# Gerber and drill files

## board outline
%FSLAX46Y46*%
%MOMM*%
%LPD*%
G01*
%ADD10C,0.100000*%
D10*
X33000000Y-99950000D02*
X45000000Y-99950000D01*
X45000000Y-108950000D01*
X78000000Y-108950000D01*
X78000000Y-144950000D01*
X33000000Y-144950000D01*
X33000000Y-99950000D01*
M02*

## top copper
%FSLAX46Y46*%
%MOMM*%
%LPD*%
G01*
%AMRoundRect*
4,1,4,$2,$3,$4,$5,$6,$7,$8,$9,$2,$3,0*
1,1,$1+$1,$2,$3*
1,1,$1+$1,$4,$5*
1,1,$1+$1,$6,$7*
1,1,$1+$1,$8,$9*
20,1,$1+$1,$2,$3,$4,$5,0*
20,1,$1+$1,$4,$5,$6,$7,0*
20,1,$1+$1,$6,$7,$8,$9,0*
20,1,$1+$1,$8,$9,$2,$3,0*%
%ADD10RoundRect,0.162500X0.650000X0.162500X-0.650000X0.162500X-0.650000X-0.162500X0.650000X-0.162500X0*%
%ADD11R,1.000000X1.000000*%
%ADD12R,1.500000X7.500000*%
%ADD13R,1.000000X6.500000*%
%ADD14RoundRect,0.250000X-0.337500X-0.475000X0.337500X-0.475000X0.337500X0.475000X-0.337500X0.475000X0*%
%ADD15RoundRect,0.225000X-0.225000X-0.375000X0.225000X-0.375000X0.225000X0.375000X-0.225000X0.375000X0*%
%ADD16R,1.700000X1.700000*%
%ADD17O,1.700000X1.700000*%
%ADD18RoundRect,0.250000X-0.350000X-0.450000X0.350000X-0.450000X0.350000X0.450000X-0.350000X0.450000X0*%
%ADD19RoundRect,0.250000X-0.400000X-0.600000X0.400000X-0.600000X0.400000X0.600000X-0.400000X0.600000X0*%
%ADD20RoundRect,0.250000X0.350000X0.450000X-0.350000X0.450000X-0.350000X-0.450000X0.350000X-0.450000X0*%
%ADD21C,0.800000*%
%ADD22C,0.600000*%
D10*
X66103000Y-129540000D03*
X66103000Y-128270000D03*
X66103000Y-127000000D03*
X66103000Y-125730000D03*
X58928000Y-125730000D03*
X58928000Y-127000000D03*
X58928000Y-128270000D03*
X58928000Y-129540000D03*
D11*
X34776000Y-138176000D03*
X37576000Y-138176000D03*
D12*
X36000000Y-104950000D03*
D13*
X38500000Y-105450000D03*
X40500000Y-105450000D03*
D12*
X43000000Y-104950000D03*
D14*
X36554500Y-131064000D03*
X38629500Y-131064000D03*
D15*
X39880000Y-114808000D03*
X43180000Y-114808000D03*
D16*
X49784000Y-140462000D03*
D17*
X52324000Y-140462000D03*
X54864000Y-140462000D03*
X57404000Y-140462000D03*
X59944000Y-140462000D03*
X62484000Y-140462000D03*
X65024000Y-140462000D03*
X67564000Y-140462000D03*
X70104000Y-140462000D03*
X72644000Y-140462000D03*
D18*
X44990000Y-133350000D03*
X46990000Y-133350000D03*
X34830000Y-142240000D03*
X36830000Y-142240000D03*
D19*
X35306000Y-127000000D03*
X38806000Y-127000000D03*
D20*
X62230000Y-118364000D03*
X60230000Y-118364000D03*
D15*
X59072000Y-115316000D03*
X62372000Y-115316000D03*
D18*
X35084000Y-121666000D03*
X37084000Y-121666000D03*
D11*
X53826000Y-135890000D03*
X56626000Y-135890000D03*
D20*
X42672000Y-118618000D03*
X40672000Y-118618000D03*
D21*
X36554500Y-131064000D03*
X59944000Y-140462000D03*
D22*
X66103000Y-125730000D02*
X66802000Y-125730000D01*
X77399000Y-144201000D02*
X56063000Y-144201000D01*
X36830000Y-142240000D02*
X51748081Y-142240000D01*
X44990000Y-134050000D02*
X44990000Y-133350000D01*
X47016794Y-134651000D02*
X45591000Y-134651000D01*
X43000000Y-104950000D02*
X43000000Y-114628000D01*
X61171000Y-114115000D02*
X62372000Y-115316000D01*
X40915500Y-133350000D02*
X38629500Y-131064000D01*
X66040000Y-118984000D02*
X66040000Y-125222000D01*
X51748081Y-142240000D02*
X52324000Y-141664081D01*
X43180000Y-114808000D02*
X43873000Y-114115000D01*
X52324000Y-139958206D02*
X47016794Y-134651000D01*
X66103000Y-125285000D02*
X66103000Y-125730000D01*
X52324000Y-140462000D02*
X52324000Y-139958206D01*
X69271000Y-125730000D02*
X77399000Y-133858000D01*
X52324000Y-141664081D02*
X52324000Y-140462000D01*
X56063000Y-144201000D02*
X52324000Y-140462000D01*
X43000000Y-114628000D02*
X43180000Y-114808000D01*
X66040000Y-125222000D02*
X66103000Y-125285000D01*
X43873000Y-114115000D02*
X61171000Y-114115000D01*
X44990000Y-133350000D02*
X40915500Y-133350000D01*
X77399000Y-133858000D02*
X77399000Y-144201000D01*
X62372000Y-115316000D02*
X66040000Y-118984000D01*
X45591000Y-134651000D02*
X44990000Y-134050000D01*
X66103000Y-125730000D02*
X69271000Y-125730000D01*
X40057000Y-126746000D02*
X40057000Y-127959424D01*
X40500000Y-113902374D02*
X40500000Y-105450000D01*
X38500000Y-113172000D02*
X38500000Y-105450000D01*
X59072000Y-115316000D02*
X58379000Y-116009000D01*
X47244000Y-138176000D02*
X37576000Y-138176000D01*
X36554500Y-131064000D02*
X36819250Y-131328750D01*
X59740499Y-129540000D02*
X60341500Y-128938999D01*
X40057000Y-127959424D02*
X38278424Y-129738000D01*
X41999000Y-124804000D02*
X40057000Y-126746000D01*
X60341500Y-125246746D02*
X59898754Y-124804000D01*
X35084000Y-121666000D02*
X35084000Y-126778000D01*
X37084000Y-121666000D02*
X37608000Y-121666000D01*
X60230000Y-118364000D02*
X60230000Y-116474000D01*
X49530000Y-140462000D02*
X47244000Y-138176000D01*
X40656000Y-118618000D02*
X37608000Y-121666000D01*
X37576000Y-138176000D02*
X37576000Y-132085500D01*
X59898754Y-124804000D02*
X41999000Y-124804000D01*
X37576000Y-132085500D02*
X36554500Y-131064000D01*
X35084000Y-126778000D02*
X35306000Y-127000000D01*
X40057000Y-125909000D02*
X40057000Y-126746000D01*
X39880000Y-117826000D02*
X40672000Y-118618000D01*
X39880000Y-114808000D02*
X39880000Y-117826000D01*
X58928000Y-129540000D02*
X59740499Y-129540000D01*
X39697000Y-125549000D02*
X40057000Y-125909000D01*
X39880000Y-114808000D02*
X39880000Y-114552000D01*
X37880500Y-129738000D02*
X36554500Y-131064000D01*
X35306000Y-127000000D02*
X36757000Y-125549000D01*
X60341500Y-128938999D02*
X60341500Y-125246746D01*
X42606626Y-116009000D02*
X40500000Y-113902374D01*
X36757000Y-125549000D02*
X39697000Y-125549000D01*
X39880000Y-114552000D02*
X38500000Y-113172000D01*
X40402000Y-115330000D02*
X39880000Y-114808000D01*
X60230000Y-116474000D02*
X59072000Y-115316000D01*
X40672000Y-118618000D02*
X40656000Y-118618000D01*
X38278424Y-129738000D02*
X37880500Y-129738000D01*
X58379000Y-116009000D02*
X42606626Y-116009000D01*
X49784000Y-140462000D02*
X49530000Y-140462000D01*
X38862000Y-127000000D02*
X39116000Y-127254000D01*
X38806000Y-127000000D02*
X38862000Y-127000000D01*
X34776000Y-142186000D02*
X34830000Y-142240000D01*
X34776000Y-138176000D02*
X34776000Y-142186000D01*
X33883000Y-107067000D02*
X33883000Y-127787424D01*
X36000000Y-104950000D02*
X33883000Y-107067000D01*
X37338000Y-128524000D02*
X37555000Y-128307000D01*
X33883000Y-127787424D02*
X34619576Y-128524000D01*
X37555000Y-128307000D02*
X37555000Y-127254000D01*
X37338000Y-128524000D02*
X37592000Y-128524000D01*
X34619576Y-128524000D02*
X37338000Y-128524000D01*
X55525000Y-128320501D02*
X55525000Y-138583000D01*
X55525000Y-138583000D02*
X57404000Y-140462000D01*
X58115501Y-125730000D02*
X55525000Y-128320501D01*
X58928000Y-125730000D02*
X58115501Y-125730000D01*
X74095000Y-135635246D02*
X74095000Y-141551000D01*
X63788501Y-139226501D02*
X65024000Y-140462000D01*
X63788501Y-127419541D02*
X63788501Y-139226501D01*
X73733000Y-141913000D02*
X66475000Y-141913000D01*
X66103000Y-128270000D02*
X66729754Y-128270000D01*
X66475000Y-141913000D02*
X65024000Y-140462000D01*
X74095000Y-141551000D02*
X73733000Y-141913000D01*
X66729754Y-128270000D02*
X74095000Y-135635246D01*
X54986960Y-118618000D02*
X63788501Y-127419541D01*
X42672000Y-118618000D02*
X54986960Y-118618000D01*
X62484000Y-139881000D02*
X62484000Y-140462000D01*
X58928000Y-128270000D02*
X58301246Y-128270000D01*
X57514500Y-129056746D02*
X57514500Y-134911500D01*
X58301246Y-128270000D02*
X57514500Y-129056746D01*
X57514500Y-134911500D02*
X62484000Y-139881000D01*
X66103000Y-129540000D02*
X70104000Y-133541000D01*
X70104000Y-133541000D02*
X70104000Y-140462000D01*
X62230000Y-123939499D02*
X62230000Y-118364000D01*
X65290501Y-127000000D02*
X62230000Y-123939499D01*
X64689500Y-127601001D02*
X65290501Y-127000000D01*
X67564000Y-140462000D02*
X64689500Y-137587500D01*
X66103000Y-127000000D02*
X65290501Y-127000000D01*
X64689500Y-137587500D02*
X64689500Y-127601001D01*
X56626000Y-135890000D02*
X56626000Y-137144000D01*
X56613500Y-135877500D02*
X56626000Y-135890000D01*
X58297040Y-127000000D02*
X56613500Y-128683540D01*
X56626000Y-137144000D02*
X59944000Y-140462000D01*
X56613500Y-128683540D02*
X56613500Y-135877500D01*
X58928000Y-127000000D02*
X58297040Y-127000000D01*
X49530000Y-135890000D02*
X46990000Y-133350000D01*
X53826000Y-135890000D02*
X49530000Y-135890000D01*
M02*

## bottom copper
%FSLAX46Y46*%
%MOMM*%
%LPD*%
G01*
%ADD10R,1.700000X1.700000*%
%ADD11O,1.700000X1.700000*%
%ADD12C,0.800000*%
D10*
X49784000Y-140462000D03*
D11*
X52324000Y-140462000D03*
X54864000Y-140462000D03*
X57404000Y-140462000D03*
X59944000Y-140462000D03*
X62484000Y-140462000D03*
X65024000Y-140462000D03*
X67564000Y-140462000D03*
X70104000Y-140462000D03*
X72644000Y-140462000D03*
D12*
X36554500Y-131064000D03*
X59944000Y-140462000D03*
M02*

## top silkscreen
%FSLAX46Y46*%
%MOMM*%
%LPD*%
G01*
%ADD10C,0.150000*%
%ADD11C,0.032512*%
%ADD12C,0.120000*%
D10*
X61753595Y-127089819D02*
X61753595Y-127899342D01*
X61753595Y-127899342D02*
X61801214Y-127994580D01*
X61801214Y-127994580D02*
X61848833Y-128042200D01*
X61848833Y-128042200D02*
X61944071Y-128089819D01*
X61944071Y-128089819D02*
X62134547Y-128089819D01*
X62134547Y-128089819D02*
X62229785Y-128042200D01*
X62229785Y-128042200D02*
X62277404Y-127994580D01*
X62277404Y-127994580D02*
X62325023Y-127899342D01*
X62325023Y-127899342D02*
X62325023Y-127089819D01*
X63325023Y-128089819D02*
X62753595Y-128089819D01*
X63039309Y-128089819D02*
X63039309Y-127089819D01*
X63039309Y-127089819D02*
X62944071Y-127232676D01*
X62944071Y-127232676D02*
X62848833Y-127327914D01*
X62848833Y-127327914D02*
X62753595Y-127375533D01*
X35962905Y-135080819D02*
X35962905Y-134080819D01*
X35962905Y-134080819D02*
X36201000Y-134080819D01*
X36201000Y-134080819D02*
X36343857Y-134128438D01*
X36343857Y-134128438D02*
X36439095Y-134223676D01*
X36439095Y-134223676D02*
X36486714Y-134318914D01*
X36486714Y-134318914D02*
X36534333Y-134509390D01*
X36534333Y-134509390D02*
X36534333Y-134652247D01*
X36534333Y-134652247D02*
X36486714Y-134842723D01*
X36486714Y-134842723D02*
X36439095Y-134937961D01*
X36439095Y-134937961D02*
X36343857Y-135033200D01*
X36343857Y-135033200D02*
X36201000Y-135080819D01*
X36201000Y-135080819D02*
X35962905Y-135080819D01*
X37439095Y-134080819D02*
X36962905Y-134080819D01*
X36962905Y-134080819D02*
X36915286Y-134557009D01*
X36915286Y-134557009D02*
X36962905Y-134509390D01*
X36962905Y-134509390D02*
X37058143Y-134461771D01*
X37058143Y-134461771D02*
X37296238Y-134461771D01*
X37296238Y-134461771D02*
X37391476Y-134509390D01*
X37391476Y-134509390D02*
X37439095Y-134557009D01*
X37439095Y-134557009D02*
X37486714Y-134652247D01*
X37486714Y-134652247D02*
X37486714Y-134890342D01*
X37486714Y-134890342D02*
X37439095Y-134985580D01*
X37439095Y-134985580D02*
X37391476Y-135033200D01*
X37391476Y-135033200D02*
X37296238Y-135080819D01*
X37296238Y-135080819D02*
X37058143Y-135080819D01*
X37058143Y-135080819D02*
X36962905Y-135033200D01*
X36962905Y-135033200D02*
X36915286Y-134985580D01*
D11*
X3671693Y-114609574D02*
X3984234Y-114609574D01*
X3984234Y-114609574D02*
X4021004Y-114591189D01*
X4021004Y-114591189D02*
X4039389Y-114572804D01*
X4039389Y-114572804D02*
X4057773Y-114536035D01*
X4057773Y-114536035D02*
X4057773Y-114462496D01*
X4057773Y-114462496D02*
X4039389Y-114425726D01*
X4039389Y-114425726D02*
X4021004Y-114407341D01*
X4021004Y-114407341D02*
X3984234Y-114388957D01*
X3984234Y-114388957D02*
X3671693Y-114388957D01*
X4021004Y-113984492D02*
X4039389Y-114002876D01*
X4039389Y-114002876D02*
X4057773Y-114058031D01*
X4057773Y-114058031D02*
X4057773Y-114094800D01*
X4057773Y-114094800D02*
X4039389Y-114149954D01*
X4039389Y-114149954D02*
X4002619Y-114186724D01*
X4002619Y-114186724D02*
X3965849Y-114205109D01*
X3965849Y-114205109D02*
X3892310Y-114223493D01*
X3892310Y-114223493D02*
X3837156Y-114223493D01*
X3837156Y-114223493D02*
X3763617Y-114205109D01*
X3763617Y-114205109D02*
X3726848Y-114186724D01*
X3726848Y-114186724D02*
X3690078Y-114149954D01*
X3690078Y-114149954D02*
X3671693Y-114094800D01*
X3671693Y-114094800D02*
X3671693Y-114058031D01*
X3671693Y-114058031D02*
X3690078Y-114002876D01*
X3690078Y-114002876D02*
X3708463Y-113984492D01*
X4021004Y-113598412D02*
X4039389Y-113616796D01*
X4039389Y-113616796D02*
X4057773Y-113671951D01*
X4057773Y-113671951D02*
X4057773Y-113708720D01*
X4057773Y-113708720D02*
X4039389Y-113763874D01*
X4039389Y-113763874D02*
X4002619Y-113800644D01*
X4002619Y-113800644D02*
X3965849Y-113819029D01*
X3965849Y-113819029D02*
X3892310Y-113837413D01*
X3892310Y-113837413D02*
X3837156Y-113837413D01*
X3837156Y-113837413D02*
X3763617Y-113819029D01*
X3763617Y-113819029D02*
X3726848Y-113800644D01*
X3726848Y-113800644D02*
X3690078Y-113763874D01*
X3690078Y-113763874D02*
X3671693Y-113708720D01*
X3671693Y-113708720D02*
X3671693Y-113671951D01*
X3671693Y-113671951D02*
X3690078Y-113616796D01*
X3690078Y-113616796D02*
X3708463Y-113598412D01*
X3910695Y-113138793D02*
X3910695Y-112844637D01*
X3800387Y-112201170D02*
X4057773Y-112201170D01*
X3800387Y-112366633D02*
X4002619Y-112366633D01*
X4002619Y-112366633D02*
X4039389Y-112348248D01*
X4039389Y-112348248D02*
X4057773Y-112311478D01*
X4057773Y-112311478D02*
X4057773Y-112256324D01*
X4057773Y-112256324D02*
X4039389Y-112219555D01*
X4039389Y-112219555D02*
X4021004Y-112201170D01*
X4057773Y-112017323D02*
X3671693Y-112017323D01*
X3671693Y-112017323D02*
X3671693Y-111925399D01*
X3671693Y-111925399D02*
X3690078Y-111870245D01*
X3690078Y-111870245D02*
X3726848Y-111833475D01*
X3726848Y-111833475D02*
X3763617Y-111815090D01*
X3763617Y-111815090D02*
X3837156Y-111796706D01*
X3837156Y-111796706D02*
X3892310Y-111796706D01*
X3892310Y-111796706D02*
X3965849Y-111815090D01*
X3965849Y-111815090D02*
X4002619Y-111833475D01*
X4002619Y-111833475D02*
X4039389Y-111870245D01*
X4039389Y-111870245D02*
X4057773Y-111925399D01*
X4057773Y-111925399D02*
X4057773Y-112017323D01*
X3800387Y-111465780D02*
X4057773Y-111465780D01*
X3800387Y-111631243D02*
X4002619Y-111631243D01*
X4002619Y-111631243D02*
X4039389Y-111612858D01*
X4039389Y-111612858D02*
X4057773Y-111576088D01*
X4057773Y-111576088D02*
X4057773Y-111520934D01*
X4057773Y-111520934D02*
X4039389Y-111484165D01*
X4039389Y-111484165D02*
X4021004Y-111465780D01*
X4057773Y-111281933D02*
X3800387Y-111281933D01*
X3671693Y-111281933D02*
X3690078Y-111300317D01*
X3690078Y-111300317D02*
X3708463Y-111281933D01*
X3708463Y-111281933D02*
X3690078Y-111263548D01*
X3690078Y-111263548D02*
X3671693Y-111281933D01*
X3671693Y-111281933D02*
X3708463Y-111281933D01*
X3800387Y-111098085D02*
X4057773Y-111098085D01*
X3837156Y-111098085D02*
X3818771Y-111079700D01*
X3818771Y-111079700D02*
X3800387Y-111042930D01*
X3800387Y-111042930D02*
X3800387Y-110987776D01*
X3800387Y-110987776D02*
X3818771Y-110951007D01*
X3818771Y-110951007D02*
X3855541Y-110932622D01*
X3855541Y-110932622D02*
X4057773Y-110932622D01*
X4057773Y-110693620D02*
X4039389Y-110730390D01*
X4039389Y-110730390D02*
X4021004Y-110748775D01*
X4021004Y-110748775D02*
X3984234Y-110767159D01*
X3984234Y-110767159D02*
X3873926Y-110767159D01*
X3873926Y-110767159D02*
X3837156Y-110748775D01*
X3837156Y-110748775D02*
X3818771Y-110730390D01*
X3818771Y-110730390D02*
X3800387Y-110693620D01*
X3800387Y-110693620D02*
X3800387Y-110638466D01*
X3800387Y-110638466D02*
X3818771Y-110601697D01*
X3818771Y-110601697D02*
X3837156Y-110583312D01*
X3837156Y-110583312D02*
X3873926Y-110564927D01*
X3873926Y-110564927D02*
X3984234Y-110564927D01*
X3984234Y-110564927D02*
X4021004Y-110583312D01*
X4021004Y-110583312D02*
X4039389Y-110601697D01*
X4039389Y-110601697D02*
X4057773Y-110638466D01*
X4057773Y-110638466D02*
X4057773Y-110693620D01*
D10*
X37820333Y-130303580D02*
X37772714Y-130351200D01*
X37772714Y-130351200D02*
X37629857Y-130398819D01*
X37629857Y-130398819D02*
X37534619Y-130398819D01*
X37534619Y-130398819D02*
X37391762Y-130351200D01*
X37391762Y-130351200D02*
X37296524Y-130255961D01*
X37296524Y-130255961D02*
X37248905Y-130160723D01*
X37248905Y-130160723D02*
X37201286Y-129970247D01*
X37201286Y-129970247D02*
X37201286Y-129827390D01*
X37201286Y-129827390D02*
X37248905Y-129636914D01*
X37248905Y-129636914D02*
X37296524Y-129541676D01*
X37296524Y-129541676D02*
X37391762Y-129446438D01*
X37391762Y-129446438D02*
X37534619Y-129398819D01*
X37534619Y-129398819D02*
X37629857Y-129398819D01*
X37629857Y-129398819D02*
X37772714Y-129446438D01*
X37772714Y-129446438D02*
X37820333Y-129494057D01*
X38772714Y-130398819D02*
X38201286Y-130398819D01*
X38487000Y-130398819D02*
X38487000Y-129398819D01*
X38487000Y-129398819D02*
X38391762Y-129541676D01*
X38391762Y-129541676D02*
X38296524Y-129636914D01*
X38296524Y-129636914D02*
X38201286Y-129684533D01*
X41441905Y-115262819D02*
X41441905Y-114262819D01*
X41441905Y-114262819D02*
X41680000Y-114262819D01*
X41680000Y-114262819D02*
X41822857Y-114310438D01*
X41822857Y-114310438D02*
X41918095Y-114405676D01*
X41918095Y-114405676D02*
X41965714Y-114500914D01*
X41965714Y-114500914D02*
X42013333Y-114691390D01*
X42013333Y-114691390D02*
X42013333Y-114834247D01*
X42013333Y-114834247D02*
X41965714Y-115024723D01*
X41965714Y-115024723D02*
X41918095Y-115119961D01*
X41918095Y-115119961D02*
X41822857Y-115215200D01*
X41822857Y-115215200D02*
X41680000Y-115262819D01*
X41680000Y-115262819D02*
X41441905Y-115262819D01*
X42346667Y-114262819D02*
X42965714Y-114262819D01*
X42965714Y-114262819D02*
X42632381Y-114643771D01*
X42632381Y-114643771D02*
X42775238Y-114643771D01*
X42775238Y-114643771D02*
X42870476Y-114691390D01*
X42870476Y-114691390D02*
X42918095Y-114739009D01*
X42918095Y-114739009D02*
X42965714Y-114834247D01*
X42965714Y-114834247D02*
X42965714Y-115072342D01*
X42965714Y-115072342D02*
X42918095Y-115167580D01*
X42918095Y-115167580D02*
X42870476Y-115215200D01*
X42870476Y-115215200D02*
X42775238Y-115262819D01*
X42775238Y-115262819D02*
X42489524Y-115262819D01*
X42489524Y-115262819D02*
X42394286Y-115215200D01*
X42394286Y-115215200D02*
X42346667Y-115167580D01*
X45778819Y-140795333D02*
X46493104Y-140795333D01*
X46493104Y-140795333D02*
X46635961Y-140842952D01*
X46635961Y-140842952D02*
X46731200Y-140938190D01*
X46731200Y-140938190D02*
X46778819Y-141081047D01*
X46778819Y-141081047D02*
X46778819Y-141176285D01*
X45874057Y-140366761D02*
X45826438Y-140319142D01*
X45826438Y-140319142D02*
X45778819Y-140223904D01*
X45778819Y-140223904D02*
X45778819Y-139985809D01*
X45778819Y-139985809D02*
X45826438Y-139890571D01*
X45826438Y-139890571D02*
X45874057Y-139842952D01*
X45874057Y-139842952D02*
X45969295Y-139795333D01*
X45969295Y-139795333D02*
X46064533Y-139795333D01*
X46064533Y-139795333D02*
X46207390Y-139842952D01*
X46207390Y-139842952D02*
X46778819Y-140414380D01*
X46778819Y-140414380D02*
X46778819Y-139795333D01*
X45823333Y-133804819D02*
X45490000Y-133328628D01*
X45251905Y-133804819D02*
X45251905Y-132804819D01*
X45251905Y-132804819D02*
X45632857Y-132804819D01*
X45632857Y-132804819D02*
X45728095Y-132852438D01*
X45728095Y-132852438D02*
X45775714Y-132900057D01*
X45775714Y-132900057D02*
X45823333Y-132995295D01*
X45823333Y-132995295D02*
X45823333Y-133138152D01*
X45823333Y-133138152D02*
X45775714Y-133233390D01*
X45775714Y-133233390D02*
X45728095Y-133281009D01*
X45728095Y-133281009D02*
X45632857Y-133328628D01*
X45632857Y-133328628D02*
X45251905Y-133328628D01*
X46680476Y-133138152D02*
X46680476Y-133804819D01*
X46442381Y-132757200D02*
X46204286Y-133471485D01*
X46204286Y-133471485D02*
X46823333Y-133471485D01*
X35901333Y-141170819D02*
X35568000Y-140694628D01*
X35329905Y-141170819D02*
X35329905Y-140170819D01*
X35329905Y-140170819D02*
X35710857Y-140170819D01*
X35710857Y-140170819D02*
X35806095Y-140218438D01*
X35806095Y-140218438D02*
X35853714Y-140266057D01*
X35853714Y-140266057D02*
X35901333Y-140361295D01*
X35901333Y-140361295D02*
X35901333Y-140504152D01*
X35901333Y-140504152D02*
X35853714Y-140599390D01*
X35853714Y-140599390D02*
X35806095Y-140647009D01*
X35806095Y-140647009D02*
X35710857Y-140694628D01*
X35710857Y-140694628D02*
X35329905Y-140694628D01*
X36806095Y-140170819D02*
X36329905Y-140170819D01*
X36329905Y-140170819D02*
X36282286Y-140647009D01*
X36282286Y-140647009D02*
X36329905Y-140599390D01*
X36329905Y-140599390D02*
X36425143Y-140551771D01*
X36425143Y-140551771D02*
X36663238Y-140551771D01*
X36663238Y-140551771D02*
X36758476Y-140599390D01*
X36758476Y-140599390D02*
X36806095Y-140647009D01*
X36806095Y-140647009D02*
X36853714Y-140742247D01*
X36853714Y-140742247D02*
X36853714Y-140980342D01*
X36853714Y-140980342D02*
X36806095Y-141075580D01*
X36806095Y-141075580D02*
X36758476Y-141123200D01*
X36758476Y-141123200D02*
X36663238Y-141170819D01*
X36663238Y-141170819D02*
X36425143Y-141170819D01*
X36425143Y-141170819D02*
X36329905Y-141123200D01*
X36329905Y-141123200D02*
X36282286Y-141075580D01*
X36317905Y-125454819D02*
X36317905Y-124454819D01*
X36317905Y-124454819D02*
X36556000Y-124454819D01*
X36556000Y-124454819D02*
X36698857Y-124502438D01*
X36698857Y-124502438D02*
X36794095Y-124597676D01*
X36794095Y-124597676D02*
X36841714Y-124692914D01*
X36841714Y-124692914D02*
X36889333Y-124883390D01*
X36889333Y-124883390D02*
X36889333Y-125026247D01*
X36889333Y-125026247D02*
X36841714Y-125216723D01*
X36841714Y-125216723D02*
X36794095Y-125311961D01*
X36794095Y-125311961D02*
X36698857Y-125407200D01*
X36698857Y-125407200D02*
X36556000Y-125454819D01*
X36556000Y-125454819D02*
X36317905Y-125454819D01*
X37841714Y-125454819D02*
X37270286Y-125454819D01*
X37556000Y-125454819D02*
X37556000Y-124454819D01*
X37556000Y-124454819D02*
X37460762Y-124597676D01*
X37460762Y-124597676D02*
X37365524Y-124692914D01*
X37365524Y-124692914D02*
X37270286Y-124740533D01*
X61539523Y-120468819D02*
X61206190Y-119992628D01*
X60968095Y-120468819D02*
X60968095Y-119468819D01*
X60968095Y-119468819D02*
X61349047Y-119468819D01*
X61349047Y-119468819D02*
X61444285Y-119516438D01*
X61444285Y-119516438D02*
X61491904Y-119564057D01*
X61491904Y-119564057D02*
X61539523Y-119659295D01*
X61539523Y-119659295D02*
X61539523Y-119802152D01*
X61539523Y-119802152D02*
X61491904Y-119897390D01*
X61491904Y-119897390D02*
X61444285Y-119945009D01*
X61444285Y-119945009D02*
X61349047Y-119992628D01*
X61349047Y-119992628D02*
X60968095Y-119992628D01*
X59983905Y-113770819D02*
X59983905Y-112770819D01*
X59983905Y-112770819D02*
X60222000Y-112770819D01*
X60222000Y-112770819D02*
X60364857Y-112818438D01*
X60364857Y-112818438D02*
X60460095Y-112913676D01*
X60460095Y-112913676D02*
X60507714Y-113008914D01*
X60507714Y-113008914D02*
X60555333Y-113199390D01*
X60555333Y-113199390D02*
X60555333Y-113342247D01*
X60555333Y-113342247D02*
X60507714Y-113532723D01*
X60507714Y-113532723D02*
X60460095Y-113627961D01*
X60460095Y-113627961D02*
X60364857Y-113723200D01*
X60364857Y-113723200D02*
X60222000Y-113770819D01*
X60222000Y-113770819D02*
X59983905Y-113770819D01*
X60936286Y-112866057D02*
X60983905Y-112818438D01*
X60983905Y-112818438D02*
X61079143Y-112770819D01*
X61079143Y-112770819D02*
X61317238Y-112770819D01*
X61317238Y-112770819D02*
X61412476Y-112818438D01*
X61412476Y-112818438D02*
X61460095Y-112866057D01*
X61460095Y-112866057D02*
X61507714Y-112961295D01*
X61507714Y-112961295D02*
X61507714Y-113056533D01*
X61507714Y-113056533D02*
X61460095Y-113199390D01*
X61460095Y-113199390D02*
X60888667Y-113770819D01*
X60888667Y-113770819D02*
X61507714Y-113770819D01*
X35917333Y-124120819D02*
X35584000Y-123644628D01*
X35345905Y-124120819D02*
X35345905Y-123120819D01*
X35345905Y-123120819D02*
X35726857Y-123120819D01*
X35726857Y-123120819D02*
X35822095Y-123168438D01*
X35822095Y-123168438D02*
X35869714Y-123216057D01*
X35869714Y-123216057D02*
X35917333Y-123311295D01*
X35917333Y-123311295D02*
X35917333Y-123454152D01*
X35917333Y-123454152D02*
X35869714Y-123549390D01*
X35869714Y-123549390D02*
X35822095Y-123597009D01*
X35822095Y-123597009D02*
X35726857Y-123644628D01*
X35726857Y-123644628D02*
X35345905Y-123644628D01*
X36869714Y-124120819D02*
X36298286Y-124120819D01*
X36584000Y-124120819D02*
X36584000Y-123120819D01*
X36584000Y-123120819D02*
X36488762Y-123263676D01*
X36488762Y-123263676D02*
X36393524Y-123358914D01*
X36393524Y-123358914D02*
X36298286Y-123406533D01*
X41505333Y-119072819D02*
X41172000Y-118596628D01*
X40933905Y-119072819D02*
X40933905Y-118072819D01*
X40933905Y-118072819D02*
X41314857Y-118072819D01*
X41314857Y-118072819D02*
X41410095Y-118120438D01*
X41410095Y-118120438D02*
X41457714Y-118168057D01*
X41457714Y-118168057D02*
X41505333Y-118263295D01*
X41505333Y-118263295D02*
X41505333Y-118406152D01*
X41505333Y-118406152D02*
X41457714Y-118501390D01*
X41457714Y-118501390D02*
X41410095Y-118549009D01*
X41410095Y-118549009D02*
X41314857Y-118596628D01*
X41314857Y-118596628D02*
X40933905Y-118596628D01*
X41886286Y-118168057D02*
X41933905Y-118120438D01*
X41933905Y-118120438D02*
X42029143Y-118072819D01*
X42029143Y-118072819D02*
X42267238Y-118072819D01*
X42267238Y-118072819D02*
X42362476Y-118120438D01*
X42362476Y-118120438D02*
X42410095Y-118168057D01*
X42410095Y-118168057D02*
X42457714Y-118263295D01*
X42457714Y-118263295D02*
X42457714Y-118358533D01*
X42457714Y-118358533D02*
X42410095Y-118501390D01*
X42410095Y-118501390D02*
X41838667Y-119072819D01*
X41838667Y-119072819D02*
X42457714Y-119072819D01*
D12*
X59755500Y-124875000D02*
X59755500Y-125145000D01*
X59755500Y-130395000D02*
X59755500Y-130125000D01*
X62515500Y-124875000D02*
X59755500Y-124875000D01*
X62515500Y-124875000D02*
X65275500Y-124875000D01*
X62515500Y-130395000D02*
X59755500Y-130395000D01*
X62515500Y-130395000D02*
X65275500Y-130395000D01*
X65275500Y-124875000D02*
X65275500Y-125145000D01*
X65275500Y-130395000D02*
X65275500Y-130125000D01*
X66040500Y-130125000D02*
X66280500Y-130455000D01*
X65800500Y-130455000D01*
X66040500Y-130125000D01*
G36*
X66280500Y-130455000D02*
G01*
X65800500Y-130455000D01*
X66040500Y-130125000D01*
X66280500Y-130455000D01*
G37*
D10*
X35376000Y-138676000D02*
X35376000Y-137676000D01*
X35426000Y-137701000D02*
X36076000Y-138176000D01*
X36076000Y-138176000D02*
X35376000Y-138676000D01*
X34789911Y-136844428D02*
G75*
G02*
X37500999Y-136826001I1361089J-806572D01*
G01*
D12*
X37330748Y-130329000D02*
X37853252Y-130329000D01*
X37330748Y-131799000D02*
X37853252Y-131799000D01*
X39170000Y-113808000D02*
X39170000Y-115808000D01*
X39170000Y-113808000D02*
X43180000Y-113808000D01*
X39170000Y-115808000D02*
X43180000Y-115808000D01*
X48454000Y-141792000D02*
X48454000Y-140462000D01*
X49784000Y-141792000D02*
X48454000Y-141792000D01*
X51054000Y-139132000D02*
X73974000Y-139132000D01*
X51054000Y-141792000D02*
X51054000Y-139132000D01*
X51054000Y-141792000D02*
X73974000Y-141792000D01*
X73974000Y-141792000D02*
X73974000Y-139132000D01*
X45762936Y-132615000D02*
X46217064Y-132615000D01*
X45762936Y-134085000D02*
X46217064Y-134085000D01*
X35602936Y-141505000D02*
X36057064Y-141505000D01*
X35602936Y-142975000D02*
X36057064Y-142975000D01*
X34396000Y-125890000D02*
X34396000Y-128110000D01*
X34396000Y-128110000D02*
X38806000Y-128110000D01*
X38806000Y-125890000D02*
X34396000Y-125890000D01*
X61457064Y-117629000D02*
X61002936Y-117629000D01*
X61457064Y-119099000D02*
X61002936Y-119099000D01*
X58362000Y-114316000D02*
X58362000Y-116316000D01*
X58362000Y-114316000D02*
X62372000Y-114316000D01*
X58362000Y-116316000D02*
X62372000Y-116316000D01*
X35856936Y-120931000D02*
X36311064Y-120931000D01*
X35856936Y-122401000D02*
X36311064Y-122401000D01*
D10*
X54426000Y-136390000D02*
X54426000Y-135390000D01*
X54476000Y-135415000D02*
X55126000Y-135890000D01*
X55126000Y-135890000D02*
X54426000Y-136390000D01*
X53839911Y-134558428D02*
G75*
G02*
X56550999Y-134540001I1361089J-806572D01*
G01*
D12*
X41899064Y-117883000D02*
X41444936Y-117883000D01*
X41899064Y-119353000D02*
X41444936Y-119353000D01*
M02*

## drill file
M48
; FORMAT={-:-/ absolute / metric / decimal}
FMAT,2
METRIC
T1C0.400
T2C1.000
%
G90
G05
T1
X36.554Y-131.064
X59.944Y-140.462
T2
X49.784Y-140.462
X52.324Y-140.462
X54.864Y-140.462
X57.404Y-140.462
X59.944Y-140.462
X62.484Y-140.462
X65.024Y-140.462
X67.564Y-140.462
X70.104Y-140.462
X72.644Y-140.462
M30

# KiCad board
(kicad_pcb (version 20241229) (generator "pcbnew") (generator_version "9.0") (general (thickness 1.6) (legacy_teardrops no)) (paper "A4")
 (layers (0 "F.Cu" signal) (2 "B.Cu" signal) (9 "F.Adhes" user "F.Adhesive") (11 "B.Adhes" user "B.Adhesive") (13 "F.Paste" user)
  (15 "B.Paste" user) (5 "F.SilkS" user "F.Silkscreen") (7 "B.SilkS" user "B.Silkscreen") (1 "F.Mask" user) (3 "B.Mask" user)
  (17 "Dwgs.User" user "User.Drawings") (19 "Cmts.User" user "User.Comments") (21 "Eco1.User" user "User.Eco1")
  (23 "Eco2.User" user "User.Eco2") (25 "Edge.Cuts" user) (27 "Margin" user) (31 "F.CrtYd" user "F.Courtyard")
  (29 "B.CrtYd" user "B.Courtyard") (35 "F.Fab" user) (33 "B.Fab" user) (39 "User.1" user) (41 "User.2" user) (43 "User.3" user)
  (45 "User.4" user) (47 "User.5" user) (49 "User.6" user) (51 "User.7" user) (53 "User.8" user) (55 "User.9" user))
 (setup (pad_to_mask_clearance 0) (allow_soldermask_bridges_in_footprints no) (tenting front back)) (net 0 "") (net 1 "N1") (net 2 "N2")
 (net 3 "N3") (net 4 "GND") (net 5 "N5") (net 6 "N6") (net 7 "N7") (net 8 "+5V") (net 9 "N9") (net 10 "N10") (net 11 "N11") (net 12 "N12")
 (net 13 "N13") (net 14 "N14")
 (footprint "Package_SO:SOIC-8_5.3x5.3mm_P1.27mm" (layer "F.Cu") (at 62.5155 127.635 180)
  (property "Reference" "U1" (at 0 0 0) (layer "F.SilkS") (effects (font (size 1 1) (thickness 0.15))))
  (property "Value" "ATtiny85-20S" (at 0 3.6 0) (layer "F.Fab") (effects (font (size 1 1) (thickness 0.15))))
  (fp_line (start 2.76 2.76) (end 2.76 2.49) (stroke (width 0.12) (type solid)) (layer "F.SilkS"))
  (fp_line (start 2.76 -2.76) (end 2.76 -2.49) (stroke (width 0.12) (type solid)) (layer "F.SilkS"))
  (fp_line (start 0 2.76) (end 2.76 2.76) (stroke (width 0.12) (type solid)) (layer "F.SilkS"))
  (fp_line (start 0 2.76) (end -2.76 2.76) (stroke (width 0.12) (type solid)) (layer "F.SilkS"))
  (fp_line (start 0 -2.76) (end 2.76 -2.76) (stroke (width 0.12) (type solid)) (layer "F.SilkS"))
  (fp_line (start 0 -2.76) (end -2.76 -2.76) (stroke (width 0.12) (type solid)) (layer "F.SilkS"))
  (fp_line (start -2.76 2.76) (end -2.76 2.49) (stroke (width 0.12) (type solid)) (layer "F.SilkS"))
  (fp_line (start -2.76 -2.76) (end -2.76 -2.49) (stroke (width 0.12) (type solid)) (layer "F.SilkS"))
  (fp_poly
   (pts (xy -3.525 -2.49) (xy -3.765 -2.82) (xy -3.285 -2.82) (xy -3.525 -2.49)) (stroke (width 0.12) (type solid)) (fill yes)
   (layer "F.SilkS"))
  (pad "1" smd roundrect (at -3.5875 -1.905 180) (size 1.625 0.65) (layers "F.Cu" "F.Mask" "F.Paste") (roundrect_rratio 0.25) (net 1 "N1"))
  (pad "2" smd roundrect (at -3.5875 -0.635 180) (size 1.625 0.65) (layers "F.Cu" "F.Mask" "F.Paste") (roundrect_rratio 0.25) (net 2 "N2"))
  (pad "3" smd roundrect (at -3.5875 0.635 180) (size 1.625 0.65) (layers "F.Cu" "F.Mask" "F.Paste") (roundrect_rratio 0.25) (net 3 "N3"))
  (pad "4" smd roundrect (at -3.5875 1.905 180) (size 1.625 0.65) (layers "F.Cu" "F.Mask" "F.Paste") (roundrect_rratio 0.25) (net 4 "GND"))
  (pad "5" smd roundrect (at 3.5875 1.905 180) (size 1.625 0.65) (layers "F.Cu" "F.Mask" "F.Paste") (roundrect_rratio 0.25) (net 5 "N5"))
  (pad "6" smd roundrect (at 3.5875 0.635 180) (size 1.625 0.65) (layers "F.Cu" "F.Mask" "F.Paste") (roundrect_rratio 0.25) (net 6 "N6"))
  (pad "7" smd roundrect (at 3.5875 -0.635 180) (size 1.625 0.65) (layers "F.Cu" "F.Mask" "F.Paste") (roundrect_rratio 0.25) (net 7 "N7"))
  (pad "8" smd roundrect (at 3.5875 -1.905 180) (size 1.625 0.65) (layers "F.Cu" "F.Mask" "F.Paste") (roundrect_rratio 0.25) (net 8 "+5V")))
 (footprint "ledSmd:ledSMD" (layer "F.Cu") (at 36.576 138.176)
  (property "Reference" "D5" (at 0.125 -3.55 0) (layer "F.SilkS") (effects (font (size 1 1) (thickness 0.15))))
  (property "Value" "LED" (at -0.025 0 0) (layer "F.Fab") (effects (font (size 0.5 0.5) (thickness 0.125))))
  (fp_line (start -1.2 0.5) (end -1.2 -0.5) (stroke (width 0.15) (type solid)) (layer "F.SilkS"))
  (fp_line (start -1.15 -0.475) (end -0.5 0) (stroke (width 0.15) (type solid)) (layer "F.SilkS"))
  (fp_line (start -0.5 0) (end -1.2 0.5) (stroke (width 0.15) (type solid)) (layer "F.SilkS"))
  (fp_arc (start -1.786089 -1.331572) (mid -0.435753 -2.107089) (end 0.924999 -1.349999) (stroke (width 0.15) (type solid))
   (layer "F.SilkS"))
  (pad "1" smd rect (at -1.8 0) (size 1 1) (layers "F.Cu" "F.Mask" "F.Paste") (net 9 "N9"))
  (pad "2" smd rect (at 1 0) (size 1 1) (layers "F.Cu" "F.Mask" "F.Paste") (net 8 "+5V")))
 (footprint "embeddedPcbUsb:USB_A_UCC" (layer "F.Cu") (at 39.5 105.15 -90)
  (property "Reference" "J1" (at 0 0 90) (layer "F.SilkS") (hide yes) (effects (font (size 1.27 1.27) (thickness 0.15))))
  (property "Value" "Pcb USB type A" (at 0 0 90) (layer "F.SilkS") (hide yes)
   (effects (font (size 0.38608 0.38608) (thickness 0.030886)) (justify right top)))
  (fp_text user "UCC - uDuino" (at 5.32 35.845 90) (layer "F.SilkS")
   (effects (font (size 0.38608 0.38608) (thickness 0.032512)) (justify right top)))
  (pad "1" smd rect (at -0.2 3.5 270) (size 7.5 1.5) (layers "F.Cu" "F.Mask" "F.Paste") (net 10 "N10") (solder_mask_margin 0.1016))
  (pad "2" smd rect (at 0.3 1 270) (size 6.5 1) (layers "F.Cu" "F.Mask" "F.Paste") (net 8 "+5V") (solder_mask_margin 0.1016))
  (pad "3" smd rect (at 0.3 -1 270) (size 6.5 1) (layers "F.Cu" "F.Mask" "F.Paste") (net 8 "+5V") (solder_mask_margin 0.1016))
  (pad "4" smd rect (at -0.2 -3.5 270) (size 7.5 1.5) (layers "F.Cu" "F.Mask" "F.Paste") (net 4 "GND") (solder_mask_margin 0.1016)))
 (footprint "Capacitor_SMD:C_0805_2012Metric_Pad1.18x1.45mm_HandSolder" (layer "F.Cu") (at 37.592 131.064)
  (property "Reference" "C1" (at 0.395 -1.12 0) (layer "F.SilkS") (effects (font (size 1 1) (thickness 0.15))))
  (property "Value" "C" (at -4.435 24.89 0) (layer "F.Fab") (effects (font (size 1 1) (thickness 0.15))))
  (fp_line (start -0.261252 -0.735) (end 0.261252 -0.735) (stroke (width 0.12) (type solid)) (layer "F.SilkS"))
  (fp_line (start -0.261252 0.735) (end 0.261252 0.735) (stroke (width 0.12) (type solid)) (layer "F.SilkS"))
  (pad "1" smd roundrect (at -1.0375 0) (size 1.175 1.45) (layers "F.Cu" "F.Mask" "F.Paste") (roundrect_rratio 0.212766) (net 8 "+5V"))
  (pad "2" smd roundrect (at 1.0375 0) (size 1.175 1.45) (layers "F.Cu" "F.Mask" "F.Paste") (roundrect_rratio 0.212766) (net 4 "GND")))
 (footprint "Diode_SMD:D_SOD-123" (layer "F.Cu") (at 41.53 114.808)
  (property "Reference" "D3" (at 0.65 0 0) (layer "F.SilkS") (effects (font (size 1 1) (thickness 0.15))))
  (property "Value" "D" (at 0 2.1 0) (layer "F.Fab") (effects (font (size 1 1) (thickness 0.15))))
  (fp_line (start -2.36 -1) (end -2.36 1) (stroke (width 0.12) (type solid)) (layer "F.SilkS"))
  (fp_line (start -2.36 -1) (end 1.65 -1) (stroke (width 0.12) (type solid)) (layer "F.SilkS"))
  (fp_line (start -2.36 1) (end 1.65 1) (stroke (width 0.12) (type solid)) (layer "F.SilkS"))
  (pad "1" smd roundrect (at -1.65 0) (size 0.9 1.2) (layers "F.Cu" "F.Mask" "F.Paste") (roundrect_rratio 0.25) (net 8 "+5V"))
  (pad "2" smd roundrect (at 1.65 0) (size 0.9 1.2) (layers "F.Cu" "F.Mask" "F.Paste") (roundrect_rratio 0.25) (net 4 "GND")))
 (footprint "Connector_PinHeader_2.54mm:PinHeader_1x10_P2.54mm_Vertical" (layer "F.Cu") (at 49.784 140.462 90)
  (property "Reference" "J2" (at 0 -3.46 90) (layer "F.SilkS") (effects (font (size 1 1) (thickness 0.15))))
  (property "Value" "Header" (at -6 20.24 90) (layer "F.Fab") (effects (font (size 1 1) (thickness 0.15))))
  (fp_line (start -1.33 -1.33) (end 0 -1.33) (stroke (width 0.12) (type solid)) (layer "F.SilkS"))
  (fp_line (start -1.33 0) (end -1.33 -1.33) (stroke (width 0.12) (type solid)) (layer "F.SilkS"))
  (fp_line (start 1.33 1.27) (end 1.33 24.19) (stroke (width 0.12) (type solid)) (layer "F.SilkS"))
  (fp_line (start -1.33 1.27) (end 1.33 1.27) (stroke (width 0.12) (type solid)) (layer "F.SilkS"))
  (fp_line (start -1.33 1.27) (end -1.33 24.19) (stroke (width 0.12) (type solid)) (layer "F.SilkS"))
  (fp_line (start -1.33 24.19) (end 1.33 24.19) (stroke (width 0.12) (type solid)) (layer "F.SilkS"))
  (pad "1" thru_hole rect (at 0 0 90) (size 1.7 1.7) (drill 1) (layers "*.Cu" "*.Mask") (remove_unused_layers no) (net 8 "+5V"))
  (pad "2" thru_hole oval (at 0 2.54 90) (size 1.7 1.7) (drill 1) (layers "*.Cu" "*.Mask") (remove_unused_layers no) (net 4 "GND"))
  (pad "3" thru_hole oval (at 0 5.08 90) (size 1.7 1.7) (drill 1) (layers "*.Cu" "*.Mask") (remove_unused_layers no) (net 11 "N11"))
  (pad "4" thru_hole oval (at 0 7.62 90) (size 1.7 1.7) (drill 1) (layers "*.Cu" "*.Mask") (remove_unused_layers no) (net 5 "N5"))
  (pad "5" thru_hole oval (at 0 10.16 90) (size 1.7 1.7) (drill 1) (layers "*.Cu" "*.Mask") (remove_unused_layers no) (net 6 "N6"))
  (pad "6" thru_hole oval (at 0 12.7 90) (size 1.7 1.7) (drill 1) (layers "*.Cu" "*.Mask") (remove_unused_layers no) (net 7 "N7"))
  (pad "7" thru_hole oval (at 0 15.24 90) (size 1.7 1.7) (drill 1) (layers "*.Cu" "*.Mask") (remove_unused_layers no) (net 2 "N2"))
  (pad "8" thru_hole oval (at 0 17.78 90) (size 1.7 1.7) (drill 1) (layers "*.Cu" "*.Mask") (remove_unused_layers no) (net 3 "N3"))
  (pad "9" thru_hole oval (at 0 20.32 90) (size 1.7 1.7) (drill 1) (layers "*.Cu" "*.Mask") (remove_unused_layers no) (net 1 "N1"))
  (pad "10" thru_hole oval (at 0 22.86 90) (size 1.7 1.7) (drill 1) (layers "*.Cu" "*.Mask") (remove_unused_layers no) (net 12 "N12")))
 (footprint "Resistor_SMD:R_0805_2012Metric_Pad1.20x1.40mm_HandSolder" (layer "F.Cu") (at 45.99 133.35)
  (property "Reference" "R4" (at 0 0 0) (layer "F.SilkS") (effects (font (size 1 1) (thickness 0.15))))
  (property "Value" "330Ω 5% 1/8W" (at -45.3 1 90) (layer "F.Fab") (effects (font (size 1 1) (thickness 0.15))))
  (fp_line (start -0.227064 -0.735) (end 0.227064 -0.735) (stroke (width 0.12) (type solid)) (layer "F.SilkS"))
  (fp_line (start -0.227064 0.735) (end 0.227064 0.735) (stroke (width 0.12) (type solid)) (layer "F.SilkS"))
  (pad "1" smd roundrect (at -1 0) (size 1.2 1.4) (layers "F.Cu" "F.Mask" "F.Paste") (roundrect_rratio 0.208333) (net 4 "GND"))
  (pad "2" smd roundrect (at 1 0) (size 1.2 1.4) (layers "F.Cu" "F.Mask" "F.Paste") (roundrect_rratio 0.208333) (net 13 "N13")))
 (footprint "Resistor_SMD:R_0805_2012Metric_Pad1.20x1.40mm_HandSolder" (layer "F.Cu") (at 35.83 142.24)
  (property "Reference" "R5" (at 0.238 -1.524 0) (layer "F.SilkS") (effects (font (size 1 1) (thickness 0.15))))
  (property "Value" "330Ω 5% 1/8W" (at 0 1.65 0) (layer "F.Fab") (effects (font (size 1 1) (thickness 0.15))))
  (fp_line (start -0.227064 -0.735) (end 0.227064 -0.735) (stroke (width 0.12) (type solid)) (layer "F.SilkS"))
  (fp_line (start -0.227064 0.735) (end 0.227064 0.735) (stroke (width 0.12) (type solid)) (layer "F.SilkS"))
  (pad "1" smd roundrect (at -1 0) (size 1.2 1.4) (layers "F.Cu" "F.Mask" "F.Paste") (roundrect_rratio 0.208333) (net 9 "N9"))
  (pad "2" smd roundrect (at 1 0) (size 1.2 1.4) (layers "F.Cu" "F.Mask" "F.Paste") (roundrect_rratio 0.208333) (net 4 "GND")))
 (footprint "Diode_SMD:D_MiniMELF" (layer "F.Cu") (at 37.056 127)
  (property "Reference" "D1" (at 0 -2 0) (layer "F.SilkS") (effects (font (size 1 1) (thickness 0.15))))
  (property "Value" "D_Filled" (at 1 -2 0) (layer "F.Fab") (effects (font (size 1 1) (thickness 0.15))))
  (fp_line (start -2.66 -1.11) (end -2.66 1.11) (stroke (width 0.12) (type solid)) (layer "F.SilkS"))
  (fp_line (start -2.66 1.11) (end 1.75 1.11) (stroke (width 0.12) (type solid)) (layer "F.SilkS"))
  (fp_line (start 1.75 -1.11) (end -2.66 -1.11) (stroke (width 0.12) (type solid)) (layer "F.SilkS"))
  (pad "1" smd roundrect (at -1.75 0) (size 1.3 1.7) (layers "F.Cu" "F.Mask" "F.Paste") (roundrect_rratio 0.1923076923) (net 8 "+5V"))
  (pad "2" smd roundrect (at 1.75 0) (size 1.3 1.7) (layers "F.Cu" "F.Mask" "F.Paste") (roundrect_rratio 0.1923076923) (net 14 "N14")))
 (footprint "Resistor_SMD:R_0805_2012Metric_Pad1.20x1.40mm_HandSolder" (layer "F.Cu") (at 61.23 118.364 180)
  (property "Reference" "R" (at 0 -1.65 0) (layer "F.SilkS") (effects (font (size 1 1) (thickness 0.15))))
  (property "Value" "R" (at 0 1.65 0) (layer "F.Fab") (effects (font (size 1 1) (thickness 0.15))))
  (fp_line (start -0.227064 0.735) (end 0.227064 0.735) (stroke (width 0.12) (type solid)) (layer "F.SilkS"))
  (fp_line (start -0.227064 -0.735) (end 0.227064 -0.735) (stroke (width 0.12) (type solid)) (layer "F.SilkS"))
  (pad "1" smd roundrect (at -1 0 180) (size 1.2 1.4) (layers "F.Cu" "F.Mask" "F.Paste") (roundrect_rratio 0.208333) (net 3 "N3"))
  (pad "2" smd roundrect (at 1 0 180) (size 1.2 1.4) (layers "F.Cu" "F.Mask" "F.Paste") (roundrect_rratio 0.208333) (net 8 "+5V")))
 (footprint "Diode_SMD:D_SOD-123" (layer "F.Cu") (at 60.722 115.316)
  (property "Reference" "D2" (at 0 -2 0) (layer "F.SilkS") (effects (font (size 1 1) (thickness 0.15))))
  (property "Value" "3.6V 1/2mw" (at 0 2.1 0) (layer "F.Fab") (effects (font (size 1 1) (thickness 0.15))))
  (fp_line (start -2.36 -1) (end -2.36 1) (stroke (width 0.12) (type solid)) (layer "F.SilkS"))
  (fp_line (start -2.36 -1) (end 1.65 -1) (stroke (width 0.12) (type solid)) (layer "F.SilkS"))
  (fp_line (start -2.36 1) (end 1.65 1) (stroke (width 0.12) (type solid)) (layer "F.SilkS"))
  (pad "1" smd roundrect (at -1.65 0) (size 0.9 1.2) (layers "F.Cu" "F.Mask" "F.Paste") (roundrect_rratio 0.25) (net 8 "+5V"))
  (pad "2" smd roundrect (at 1.65 0) (size 0.9 1.2) (layers "F.Cu" "F.Mask" "F.Paste") (roundrect_rratio 0.25) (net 4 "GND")))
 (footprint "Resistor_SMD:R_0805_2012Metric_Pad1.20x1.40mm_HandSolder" (layer "F.Cu") (at 36.084 121.666)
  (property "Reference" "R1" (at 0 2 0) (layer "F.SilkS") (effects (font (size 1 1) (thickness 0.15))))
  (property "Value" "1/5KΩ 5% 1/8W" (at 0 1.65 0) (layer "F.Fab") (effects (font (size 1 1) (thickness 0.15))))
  (fp_line (start -0.227064 -0.735) (end 0.227064 -0.735) (stroke (width 0.12) (type solid)) (layer "F.SilkS"))
  (fp_line (start -0.227064 0.735) (end 0.227064 0.735) (stroke (width 0.12) (type solid)) (layer "F.SilkS"))
  (pad "1" smd roundrect (at -1 0) (size 1.2 1.4) (layers "F.Cu" "F.Mask" "F.Paste") (roundrect_rratio 0.208333) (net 8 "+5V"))
  (pad "2" smd roundrect (at 1 0) (size 1.2 1.4) (layers "F.Cu" "F.Mask" "F.Paste") (roundrect_rratio 0.208333) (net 8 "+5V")))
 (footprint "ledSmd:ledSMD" (layer "F.Cu") (at 55.626 135.89)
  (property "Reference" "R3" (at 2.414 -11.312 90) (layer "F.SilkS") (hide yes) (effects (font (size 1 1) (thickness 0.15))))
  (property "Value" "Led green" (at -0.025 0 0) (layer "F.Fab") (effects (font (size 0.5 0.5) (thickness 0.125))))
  (fp_line (start -1.2 0.5) (end -1.2 -0.5) (stroke (width 0.15) (type solid)) (layer "F.SilkS"))
  (fp_line (start -1.15 -0.475) (end -0.5 0) (stroke (width 0.15) (type solid)) (layer "F.SilkS"))
  (fp_line (start -0.5 0) (end -1.2 0.5) (stroke (width 0.15) (type solid)) (layer "F.SilkS"))
  (fp_arc (start -1.786089 -1.331572) (mid -0.435753 -2.107089) (end 0.924999 -1.349999) (stroke (width 0.15) (type solid))
   (layer "F.SilkS"))
  (pad "1" smd rect (at -1.8 0) (size 1 1) (layers "F.Cu" "F.Mask" "F.Paste") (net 13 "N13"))
  (pad "2" smd rect (at 1 0) (size 1 1) (layers "F.Cu" "F.Mask" "F.Paste") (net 6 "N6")))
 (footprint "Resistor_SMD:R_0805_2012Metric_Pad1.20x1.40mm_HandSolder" (layer "F.Cu") (at 41.672 118.618 180)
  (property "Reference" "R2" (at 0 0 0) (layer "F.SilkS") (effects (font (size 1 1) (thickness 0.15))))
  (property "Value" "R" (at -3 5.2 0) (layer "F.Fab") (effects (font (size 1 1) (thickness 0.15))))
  (fp_line (start -0.227064 0.735) (end 0.227064 0.735) (stroke (width 0.12) (type solid)) (layer "F.SilkS"))
  (fp_line (start -0.227064 -0.735) (end 0.227064 -0.735) (stroke (width 0.12) (type solid)) (layer "F.SilkS"))
  (pad "1" smd roundrect (at -1 0 180) (size 1.2 1.4) (layers "F.Cu" "F.Mask" "F.Paste") (roundrect_rratio 0.208333) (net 2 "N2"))
  (pad "2" smd roundrect (at 1 0 180) (size 1.2 1.4) (layers "F.Cu" "F.Mask" "F.Paste") (roundrect_rratio 0.208333) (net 8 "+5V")))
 (gr_poly
  (pts (xy 33 99.95) (xy 45 99.95) (xy 45 108.95) (xy 78 108.95) (xy 78 144.95) (xy 33 144.95)) (stroke (width 0.1) (type solid)) (fill no)
  (layer "Edge.Cuts"))
 (segment (start 66.103 125.73) (end 66.802 125.73) (width 0.6) (layer "F.Cu") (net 4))
 (segment (start 77.399 144.201) (end 56.063 144.201) (width 0.6) (layer "F.Cu") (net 4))
 (segment (start 36.83 142.24) (end 51.748081 142.24) (width 0.6) (layer "F.Cu") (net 4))
 (segment (start 44.99 134.05) (end 44.99 133.35) (width 0.6) (layer "F.Cu") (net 4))
 (segment (start 47.016794 134.651) (end 45.591 134.651) (width 0.6) (layer "F.Cu") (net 4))
 (segment (start 43 104.95) (end 43 114.628) (width 0.6) (layer "F.Cu") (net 4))
 (segment (start 61.171 114.115) (end 62.372 115.316) (width 0.6) (layer "F.Cu") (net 4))
 (segment (start 40.9155 133.35) (end 38.6295 131.064) (width 0.6) (layer "F.Cu") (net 4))
 (segment (start 66.04 118.984) (end 66.04 125.222) (width 0.6) (layer "F.Cu") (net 4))
 (segment (start 51.748081 142.24) (end 52.324 141.664081) (width 0.6) (layer "F.Cu") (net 4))
 (segment (start 43.18 114.808) (end 43.873 114.115) (width 0.6) (layer "F.Cu") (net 4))
 (segment (start 52.324 139.958206) (end 47.016794 134.651) (width 0.6) (layer "F.Cu") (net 4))
 (segment (start 66.103 125.285) (end 66.103 125.73) (width 0.6) (layer "F.Cu") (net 4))
 (segment (start 52.324 140.462) (end 52.324 139.958206) (width 0.6) (layer "F.Cu") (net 4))
 (segment (start 69.271 125.73) (end 77.399 133.858) (width 0.6) (layer "F.Cu") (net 4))
 (segment (start 52.324 141.664081) (end 52.324 140.462) (width 0.6) (layer "F.Cu") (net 4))
 (segment (start 56.063 144.201) (end 52.324 140.462) (width 0.6) (layer "F.Cu") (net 4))
 (segment (start 43 114.628) (end 43.18 114.808) (width 0.6) (layer "F.Cu") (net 4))
 (segment (start 66.04 125.222) (end 66.103 125.285) (width 0.6) (layer "F.Cu") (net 4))
 (segment (start 43.873 114.115) (end 61.171 114.115) (width 0.6) (layer "F.Cu") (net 4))
 (segment (start 44.99 133.35) (end 40.9155 133.35) (width 0.6) (layer "F.Cu") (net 4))
 (segment (start 77.399 133.858) (end 77.399 144.201) (width 0.6) (layer "F.Cu") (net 4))
 (segment (start 62.372 115.316) (end 66.04 118.984) (width 0.6) (layer "F.Cu") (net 4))
 (segment (start 45.591 134.651) (end 44.99 134.05) (width 0.6) (layer "F.Cu") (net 4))
 (segment (start 66.103 125.73) (end 69.271 125.73) (width 0.6) (layer "F.Cu") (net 4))
 (segment (start 40.057 126.746) (end 40.057 127.959424) (width 0.6) (layer "F.Cu") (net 8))
 (segment (start 40.5 113.902374) (end 40.5 105.45) (width 0.6) (layer "F.Cu") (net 8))
 (segment (start 38.5 113.172) (end 38.5 105.45) (width 0.6) (layer "F.Cu") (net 8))
 (segment (start 59.072 115.316) (end 58.379 116.009) (width 0.6) (layer "F.Cu") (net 8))
 (segment (start 47.244 138.176) (end 37.576 138.176) (width 0.6) (layer "F.Cu") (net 8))
 (segment (start 36.5545 131.064) (end 36.81925 131.32875) (width 0.6) (layer "F.Cu") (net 8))
 (segment (start 59.740499 129.54) (end 60.3415 128.938999) (width 0.6) (layer "F.Cu") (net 8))
 (segment (start 40.057 127.959424) (end 38.278424 129.738) (width 0.6) (layer "F.Cu") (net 8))
 (segment (start 41.999 124.804) (end 40.057 126.746) (width 0.6) (layer "F.Cu") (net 8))
 (segment (start 60.3415 125.246746) (end 59.898754 124.804) (width 0.6) (layer "F.Cu") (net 8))
 (segment (start 35.084 121.666) (end 35.084 126.778) (width 0.6) (layer "F.Cu") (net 8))
 (segment (start 37.084 121.666) (end 37.608 121.666) (width 0.6) (layer "F.Cu") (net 8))
 (segment (start 60.23 118.364) (end 60.23 116.474) (width 0.6) (layer "F.Cu") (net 8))
 (segment (start 49.53 140.462) (end 47.244 138.176) (width 0.6) (layer "F.Cu") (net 8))
 (segment (start 40.656 118.618) (end 37.608 121.666) (width 0.6) (layer "F.Cu") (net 8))
 (segment (start 37.576 138.176) (end 37.576 132.0855) (width 0.6) (layer "F.Cu") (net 8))
 (segment (start 59.898754 124.804) (end 41.999 124.804) (width 0.6) (layer "F.Cu") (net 8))
 (segment (start 37.576 132.0855) (end 36.5545 131.064) (width 0.6) (layer "F.Cu") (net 8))
 (segment (start 35.084 126.778) (end 35.306 127) (width 0.6) (layer "F.Cu") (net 8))
 (segment (start 40.057 125.909) (end 40.057 126.746) (width 0.6) (layer "F.Cu") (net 8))
 (segment (start 39.88 117.826) (end 40.672 118.618) (width 0.6) (layer "F.Cu") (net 8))
 (segment (start 39.88 114.808) (end 39.88 117.826) (width 0.6) (layer "F.Cu") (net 8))
 (segment (start 58.928 129.54) (end 59.740499 129.54) (width 0.6) (layer "F.Cu") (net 8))
 (segment (start 39.697 125.549) (end 40.057 125.909) (width 0.6) (layer "F.Cu") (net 8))
 (segment (start 39.88 114.808) (end 39.88 114.552) (width 0.6) (layer "F.Cu") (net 8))
 (segment (start 37.8805 129.738) (end 36.5545 131.064) (width 0.6) (layer "F.Cu") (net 8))
 (segment (start 35.306 127) (end 36.757 125.549) (width 0.6) (layer "F.Cu") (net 8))
 (segment (start 60.3415 128.938999) (end 60.3415 125.246746) (width 0.6) (layer "F.Cu") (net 8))
 (segment (start 42.606626 116.009) (end 40.5 113.902374) (width 0.6) (layer "F.Cu") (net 8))
 (segment (start 36.757 125.549) (end 39.697 125.549) (width 0.6) (layer "F.Cu") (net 8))
 (segment (start 39.88 114.552) (end 38.5 113.172) (width 0.6) (layer "F.Cu") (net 8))
 (segment (start 40.402 115.33) (end 39.88 114.808) (width 0.6) (layer "F.Cu") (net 8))
 (segment (start 60.23 116.474) (end 59.072 115.316) (width 0.6) (layer "F.Cu") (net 8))
 (segment (start 40.672 118.618) (end 40.656 118.618) (width 0.6) (layer "F.Cu") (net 8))
 (segment (start 38.278424 129.738) (end 37.8805 129.738) (width 0.6) (layer "F.Cu") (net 8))
 (segment (start 58.379 116.009) (end 42.606626 116.009) (width 0.6) (layer "F.Cu") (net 8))
 (segment (start 49.784 140.462) (end 49.53 140.462) (width 0.6) (layer "F.Cu") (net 8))
 (via (at 36.5545 131.064) (size 0.8) (drill 0.4) (layers "F.Cu" "B.Cu") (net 8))
 (segment (start 38.862 127) (end 39.116 127.254) (width 0.6) (layer "F.Cu") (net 14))
 (segment (start 38.806 127) (end 38.862 127) (width 0.6) (layer "F.Cu") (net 14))
 (segment (start 34.776 142.186) (end 34.83 142.24) (width 0.6) (layer "F.Cu") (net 9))
 (segment (start 34.776 138.176) (end 34.776 142.186) (width 0.6) (layer "F.Cu") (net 9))
 (segment (start 33.883 107.067) (end 33.883 127.787424) (width 0.6) (layer "F.Cu") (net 10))
 (segment (start 36 104.95) (end 33.883 107.067) (width 0.6) (layer "F.Cu") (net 10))
 (segment (start 37.338 128.524) (end 37.555 128.307) (width 0.6) (layer "F.Cu") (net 10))
 (segment (start 33.883 127.787424) (end 34.619576 128.524) (width 0.6) (layer "F.Cu") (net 10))
 (segment (start 37.555 128.307) (end 37.555 127.254) (width 0.6) (layer "F.Cu") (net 10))
 (segment (start 37.338 128.524) (end 37.592 128.524) (width 0.6) (layer "F.Cu") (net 10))
 (segment (start 34.619576 128.524) (end 37.338 128.524) (width 0.6) (layer "F.Cu") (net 10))
 (segment (start 55.525 128.320501) (end 55.525 138.583) (width 0.6) (layer "F.Cu") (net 5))
 (segment (start 55.525 138.583) (end 57.404 140.462) (width 0.6) (layer "F.Cu") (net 5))
 (segment (start 58.115501 125.73) (end 55.525 128.320501) (width 0.6) (layer "F.Cu") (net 5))
 (segment (start 58.928 125.73) (end 58.115501 125.73) (width 0.6) (layer "F.Cu") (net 5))
 (segment (start 74.095 135.635246) (end 74.095 141.551) (width 0.6) (layer "F.Cu") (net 2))
 (segment (start 63.788501 139.226501) (end 65.024 140.462) (width 0.6) (layer "F.Cu") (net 2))
 (segment (start 63.788501 127.419541) (end 63.788501 139.226501) (width 0.6) (layer "F.Cu") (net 2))
 (segment (start 73.733 141.913) (end 66.475 141.913) (width 0.6) (layer "F.Cu") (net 2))
 (segment (start 66.103 128.27) (end 66.729754 128.27) (width 0.6) (layer "F.Cu") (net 2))
 (segment (start 66.475 141.913) (end 65.024 140.462) (width 0.6) (layer "F.Cu") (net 2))
 (segment (start 74.095 141.551) (end 73.733 141.913) (width 0.6) (layer "F.Cu") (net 2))
 (segment (start 66.729754 128.27) (end 74.095 135.635246) (width 0.6) (layer "F.Cu") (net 2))
 (segment (start 54.98696 118.618) (end 63.788501 127.419541) (width 0.6) (layer "F.Cu") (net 2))
 (segment (start 42.672 118.618) (end 54.98696 118.618) (width 0.6) (layer "F.Cu") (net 2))
 (segment (start 62.484 139.881) (end 62.484 140.462) (width 0.6) (layer "F.Cu") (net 7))
 (segment (start 58.928 128.27) (end 58.301246 128.27) (width 0.6) (layer "F.Cu") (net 7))
 (segment (start 57.5145 129.056746) (end 57.5145 134.9115) (width 0.6) (layer "F.Cu") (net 7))
 (segment (start 58.301246 128.27) (end 57.5145 129.056746) (width 0.6) (layer "F.Cu") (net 7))
 (segment (start 57.5145 134.9115) (end 62.484 139.881) (width 0.6) (layer "F.Cu") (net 7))
 (segment (start 66.103 129.54) (end 70.104 133.541) (width 0.6) (layer "F.Cu") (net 1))
 (segment (start 70.104 133.541) (end 70.104 140.462) (width 0.6) (layer "F.Cu") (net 1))
 (segment (start 62.23 123.939499) (end 62.23 118.364) (width 0.6) (layer "F.Cu") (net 3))
 (segment (start 65.290501 127) (end 62.23 123.939499) (width 0.6) (layer "F.Cu") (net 3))
 (segment (start 64.6895 127.601001) (end 65.290501 127) (width 0.6) (layer "F.Cu") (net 3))
 (segment (start 67.564 140.462) (end 64.6895 137.5875) (width 0.6) (layer "F.Cu") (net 3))
 (segment (start 66.103 127) (end 65.290501 127) (width 0.6) (layer "F.Cu") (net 3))
 (segment (start 64.6895 137.5875) (end 64.6895 127.601001) (width 0.6) (layer "F.Cu") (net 3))
 (segment (start 56.626 135.89) (end 56.626 137.144) (width 0.6) (layer "F.Cu") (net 6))
 (segment (start 56.6135 135.8775) (end 56.626 135.89) (width 0.6) (layer "F.Cu") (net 6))
 (segment (start 58.29704 127) (end 56.6135 128.68354) (width 0.6) (layer "F.Cu") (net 6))
 (segment (start 56.626 137.144) (end 59.944 140.462) (width 0.6) (layer "F.Cu") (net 6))
 (segment (start 56.6135 128.68354) (end 56.6135 135.8775) (width 0.6) (layer "F.Cu") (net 6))
 (segment (start 58.928 127) (end 58.29704 127) (width 0.6) (layer "F.Cu") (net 6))
 (via (at 59.944 140.462) (size 0.8) (drill 0.4) (layers "F.Cu" "B.Cu") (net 6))
 (segment (start 49.53 135.89) (end 46.99 133.35) (width 0.6) (layer "F.Cu") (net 13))
 (segment (start 53.826 135.89) (end 49.53 135.89) (width 0.6) (layer "F.Cu") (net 13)))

